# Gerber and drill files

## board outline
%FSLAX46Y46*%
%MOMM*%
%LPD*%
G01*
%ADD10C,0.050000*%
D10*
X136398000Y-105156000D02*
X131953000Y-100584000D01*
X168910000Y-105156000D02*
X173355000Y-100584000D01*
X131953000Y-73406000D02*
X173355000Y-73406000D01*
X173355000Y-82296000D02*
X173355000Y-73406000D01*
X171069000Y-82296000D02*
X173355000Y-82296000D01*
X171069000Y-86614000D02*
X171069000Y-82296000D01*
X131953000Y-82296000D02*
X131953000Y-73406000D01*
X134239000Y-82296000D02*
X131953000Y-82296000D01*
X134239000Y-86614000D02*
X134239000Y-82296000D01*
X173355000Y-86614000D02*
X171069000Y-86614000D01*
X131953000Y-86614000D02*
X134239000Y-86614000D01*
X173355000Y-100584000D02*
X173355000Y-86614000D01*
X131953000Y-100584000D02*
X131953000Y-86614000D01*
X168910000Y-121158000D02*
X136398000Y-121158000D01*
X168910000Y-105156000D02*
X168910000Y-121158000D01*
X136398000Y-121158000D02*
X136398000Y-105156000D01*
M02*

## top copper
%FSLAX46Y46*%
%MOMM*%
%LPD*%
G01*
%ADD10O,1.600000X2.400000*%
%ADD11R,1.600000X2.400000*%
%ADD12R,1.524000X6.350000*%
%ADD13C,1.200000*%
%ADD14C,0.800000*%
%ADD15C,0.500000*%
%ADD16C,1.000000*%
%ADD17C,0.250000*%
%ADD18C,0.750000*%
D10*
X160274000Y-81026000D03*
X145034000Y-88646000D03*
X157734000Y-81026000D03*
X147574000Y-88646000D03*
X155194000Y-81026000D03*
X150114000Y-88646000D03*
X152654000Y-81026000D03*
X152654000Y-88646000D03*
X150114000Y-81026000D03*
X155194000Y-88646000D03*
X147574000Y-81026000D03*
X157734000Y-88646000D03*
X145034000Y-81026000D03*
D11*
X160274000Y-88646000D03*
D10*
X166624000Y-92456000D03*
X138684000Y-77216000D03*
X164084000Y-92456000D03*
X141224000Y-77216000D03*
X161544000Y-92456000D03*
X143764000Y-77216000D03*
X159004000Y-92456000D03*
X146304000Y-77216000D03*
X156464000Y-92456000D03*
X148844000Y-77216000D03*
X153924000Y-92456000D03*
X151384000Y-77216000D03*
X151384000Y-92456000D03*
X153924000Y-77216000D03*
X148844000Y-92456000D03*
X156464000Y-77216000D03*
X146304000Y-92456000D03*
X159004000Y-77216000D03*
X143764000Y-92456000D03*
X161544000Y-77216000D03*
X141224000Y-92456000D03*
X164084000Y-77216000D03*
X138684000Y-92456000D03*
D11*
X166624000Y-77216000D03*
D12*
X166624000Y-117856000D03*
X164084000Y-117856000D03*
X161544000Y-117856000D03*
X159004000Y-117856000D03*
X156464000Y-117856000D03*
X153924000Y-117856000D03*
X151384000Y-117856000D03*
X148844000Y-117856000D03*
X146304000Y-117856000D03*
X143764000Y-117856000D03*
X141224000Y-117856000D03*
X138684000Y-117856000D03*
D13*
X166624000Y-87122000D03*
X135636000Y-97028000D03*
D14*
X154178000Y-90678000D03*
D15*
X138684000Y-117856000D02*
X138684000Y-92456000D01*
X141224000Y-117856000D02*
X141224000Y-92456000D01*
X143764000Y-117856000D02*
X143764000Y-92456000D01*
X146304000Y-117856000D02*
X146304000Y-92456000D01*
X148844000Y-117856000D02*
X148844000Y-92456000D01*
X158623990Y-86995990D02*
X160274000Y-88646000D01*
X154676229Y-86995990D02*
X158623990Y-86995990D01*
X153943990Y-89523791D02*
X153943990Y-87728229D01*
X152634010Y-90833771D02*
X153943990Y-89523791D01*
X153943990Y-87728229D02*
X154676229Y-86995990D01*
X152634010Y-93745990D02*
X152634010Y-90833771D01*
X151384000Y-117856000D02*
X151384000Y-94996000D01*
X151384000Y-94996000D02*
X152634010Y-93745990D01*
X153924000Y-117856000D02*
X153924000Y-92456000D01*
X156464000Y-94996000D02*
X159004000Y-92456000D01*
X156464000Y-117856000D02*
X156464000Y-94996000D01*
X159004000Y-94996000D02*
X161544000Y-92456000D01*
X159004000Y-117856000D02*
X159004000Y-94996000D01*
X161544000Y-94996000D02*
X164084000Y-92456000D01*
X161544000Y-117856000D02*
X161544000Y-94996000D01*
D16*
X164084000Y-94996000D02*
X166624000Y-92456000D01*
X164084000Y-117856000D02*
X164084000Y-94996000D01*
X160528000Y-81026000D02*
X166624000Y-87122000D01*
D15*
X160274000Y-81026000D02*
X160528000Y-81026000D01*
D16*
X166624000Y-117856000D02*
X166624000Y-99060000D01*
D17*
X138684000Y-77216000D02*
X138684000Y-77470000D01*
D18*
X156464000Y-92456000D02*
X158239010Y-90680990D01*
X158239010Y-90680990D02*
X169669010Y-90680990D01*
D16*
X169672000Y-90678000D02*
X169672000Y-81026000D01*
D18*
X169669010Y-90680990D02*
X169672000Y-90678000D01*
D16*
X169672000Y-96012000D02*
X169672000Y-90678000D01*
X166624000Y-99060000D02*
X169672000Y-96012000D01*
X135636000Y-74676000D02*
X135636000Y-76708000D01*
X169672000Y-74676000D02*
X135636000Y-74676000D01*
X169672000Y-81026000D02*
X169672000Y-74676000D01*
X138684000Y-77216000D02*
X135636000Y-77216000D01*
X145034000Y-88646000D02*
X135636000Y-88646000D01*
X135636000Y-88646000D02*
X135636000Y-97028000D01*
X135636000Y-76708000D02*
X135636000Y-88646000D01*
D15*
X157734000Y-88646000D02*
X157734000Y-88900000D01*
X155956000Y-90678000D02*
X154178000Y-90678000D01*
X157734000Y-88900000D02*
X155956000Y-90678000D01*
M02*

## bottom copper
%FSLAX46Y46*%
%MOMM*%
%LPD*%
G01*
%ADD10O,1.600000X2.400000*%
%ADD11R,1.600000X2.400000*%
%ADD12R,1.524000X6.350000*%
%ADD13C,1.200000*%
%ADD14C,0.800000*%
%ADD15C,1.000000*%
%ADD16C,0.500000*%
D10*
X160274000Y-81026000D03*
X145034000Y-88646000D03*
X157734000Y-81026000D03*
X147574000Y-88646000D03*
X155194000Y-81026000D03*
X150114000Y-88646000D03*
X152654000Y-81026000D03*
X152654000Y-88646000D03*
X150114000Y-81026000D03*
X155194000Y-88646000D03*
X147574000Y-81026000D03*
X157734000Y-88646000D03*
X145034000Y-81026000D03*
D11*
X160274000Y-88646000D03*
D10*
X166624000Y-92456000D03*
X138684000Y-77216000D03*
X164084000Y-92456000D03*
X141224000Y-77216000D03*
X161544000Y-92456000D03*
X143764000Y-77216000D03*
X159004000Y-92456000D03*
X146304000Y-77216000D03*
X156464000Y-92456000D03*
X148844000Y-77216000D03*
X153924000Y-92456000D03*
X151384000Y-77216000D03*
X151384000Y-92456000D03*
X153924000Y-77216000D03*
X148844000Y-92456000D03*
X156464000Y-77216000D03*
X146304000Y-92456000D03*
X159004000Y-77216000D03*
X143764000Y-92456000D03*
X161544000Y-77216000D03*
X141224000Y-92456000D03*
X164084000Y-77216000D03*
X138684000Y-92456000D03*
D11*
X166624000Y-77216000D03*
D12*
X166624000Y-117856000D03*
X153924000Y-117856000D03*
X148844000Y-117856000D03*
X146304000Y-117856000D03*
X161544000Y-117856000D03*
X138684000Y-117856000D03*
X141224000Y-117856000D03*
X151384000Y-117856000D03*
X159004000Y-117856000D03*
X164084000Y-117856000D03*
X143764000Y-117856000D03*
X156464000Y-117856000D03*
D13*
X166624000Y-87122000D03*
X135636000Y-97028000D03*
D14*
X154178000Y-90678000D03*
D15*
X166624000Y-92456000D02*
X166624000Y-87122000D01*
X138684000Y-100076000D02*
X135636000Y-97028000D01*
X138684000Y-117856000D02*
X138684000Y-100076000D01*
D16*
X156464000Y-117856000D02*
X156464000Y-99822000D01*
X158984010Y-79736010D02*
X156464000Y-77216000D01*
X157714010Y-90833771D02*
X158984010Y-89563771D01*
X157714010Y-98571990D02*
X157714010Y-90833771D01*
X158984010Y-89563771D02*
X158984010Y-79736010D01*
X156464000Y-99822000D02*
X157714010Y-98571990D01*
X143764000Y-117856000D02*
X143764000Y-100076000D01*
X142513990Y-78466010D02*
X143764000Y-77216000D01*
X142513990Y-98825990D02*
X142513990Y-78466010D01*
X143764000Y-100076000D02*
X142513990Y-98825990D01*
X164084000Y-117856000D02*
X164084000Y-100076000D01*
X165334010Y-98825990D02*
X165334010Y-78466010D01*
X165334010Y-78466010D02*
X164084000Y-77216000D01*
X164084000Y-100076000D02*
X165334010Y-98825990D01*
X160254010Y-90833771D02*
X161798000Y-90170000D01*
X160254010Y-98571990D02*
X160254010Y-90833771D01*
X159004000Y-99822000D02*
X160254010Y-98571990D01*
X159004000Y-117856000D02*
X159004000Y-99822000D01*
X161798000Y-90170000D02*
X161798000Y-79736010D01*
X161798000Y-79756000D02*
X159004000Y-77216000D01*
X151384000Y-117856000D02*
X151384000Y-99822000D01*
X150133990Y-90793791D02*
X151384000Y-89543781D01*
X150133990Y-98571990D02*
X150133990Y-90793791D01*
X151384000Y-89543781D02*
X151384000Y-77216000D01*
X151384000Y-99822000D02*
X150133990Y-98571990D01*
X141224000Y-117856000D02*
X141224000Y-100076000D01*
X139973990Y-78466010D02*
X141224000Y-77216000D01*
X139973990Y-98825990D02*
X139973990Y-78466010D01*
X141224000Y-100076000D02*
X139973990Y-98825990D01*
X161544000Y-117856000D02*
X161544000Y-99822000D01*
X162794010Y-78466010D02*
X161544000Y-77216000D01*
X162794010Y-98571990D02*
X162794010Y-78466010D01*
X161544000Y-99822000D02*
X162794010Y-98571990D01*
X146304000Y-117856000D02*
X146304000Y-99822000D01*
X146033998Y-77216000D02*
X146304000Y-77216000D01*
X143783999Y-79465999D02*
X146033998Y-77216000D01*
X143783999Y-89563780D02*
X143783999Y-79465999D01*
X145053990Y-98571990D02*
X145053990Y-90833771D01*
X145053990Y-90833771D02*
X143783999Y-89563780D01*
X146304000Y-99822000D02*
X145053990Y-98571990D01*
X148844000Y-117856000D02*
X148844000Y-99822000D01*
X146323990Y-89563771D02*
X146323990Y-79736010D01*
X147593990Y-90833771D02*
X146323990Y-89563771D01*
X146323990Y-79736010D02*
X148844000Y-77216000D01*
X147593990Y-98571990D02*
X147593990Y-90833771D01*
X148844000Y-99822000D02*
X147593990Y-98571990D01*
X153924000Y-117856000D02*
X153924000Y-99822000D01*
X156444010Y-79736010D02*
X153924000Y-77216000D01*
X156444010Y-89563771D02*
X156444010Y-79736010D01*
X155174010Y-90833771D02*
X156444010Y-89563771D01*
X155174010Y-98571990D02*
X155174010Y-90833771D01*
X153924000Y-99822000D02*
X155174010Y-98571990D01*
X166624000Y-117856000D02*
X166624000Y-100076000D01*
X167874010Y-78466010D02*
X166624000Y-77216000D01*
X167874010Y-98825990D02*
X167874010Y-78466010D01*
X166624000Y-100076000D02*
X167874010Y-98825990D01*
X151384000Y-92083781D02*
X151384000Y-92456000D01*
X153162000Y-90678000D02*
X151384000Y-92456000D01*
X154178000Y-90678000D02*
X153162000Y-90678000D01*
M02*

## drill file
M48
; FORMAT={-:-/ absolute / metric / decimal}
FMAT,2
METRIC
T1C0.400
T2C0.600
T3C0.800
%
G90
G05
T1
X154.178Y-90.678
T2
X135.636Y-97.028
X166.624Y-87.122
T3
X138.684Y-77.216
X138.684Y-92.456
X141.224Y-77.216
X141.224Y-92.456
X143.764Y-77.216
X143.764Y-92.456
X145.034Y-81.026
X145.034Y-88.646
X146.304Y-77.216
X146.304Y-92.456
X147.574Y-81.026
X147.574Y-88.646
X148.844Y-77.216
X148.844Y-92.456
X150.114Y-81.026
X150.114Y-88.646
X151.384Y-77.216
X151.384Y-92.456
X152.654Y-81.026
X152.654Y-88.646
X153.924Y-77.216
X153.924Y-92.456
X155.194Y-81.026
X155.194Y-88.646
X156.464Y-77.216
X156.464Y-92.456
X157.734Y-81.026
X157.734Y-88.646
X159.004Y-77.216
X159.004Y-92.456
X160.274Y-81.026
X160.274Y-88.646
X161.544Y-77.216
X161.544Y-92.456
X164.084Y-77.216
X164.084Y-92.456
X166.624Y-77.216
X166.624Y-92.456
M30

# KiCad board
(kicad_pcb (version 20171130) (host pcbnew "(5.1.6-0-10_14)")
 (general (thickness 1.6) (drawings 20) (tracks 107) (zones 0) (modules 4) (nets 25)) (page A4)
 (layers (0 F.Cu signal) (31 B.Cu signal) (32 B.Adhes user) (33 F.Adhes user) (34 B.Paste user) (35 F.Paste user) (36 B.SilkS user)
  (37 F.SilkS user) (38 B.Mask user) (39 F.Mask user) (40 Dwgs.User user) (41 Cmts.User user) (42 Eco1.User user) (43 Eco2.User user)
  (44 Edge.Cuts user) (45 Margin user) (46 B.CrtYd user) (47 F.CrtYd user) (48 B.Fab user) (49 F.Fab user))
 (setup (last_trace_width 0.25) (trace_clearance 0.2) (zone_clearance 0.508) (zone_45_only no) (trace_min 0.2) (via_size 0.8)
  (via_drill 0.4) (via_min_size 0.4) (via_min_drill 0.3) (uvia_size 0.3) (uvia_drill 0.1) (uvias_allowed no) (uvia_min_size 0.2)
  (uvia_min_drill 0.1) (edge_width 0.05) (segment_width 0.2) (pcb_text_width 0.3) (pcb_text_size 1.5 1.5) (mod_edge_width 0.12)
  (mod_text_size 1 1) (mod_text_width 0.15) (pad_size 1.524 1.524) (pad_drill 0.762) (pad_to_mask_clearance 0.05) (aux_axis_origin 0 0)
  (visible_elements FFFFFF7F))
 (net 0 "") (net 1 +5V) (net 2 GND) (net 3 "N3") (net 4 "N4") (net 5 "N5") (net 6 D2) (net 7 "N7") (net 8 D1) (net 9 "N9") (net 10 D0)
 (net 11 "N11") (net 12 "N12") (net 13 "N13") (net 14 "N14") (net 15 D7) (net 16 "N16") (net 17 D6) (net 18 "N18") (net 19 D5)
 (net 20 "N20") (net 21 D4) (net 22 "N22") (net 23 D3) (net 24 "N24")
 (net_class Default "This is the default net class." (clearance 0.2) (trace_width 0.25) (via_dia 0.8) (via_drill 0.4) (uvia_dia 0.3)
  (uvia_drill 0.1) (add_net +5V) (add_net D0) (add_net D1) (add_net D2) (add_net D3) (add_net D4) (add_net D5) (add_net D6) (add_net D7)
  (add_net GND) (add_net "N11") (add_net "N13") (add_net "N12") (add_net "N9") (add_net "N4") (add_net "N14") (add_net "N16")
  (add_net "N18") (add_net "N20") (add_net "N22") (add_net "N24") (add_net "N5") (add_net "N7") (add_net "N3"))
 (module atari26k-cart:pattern (layer F.Cu) (at 152.654 105.41)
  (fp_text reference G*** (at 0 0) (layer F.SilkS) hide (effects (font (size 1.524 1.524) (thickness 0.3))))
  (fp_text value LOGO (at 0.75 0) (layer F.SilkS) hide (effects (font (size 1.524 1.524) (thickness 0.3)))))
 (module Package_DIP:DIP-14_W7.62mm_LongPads (layer B.Cu) (at 160.274 88.646 90)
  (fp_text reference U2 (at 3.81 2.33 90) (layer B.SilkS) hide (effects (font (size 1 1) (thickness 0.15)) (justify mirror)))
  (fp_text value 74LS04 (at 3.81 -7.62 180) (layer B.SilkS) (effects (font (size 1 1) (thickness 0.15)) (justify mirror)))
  (pad 14 thru_hole oval (at 7.62 0 90) (size 2.4 1.6) (drill 0.8) (layers *.Cu *.Mask) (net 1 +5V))
  (pad 7 thru_hole oval (at 0 -15.24 90) (size 2.4 1.6) (drill 0.8) (layers *.Cu *.Mask) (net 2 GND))
  (pad 13 thru_hole oval (at 7.62 -2.54 90) (size 2.4 1.6) (drill 0.8) (layers *.Cu *.Mask))
  (pad 6 thru_hole oval (at 0 -12.7 90) (size 2.4 1.6) (drill 0.8) (layers *.Cu *.Mask))
  (pad 12 thru_hole oval (at 7.62 -5.08 90) (size 2.4 1.6) (drill 0.8) (layers *.Cu *.Mask))
  (pad 5 thru_hole oval (at 0 -10.16 90) (size 2.4 1.6) (drill 0.8) (layers *.Cu *.Mask))
  (pad 11 thru_hole oval (at 7.62 -7.62 90) (size 2.4 1.6) (drill 0.8) (layers *.Cu *.Mask))
  (pad 4 thru_hole oval (at 0 -7.62 90) (size 2.4 1.6) (drill 0.8) (layers *.Cu *.Mask))
  (pad 10 thru_hole oval (at 7.62 -10.16 90) (size 2.4 1.6) (drill 0.8) (layers *.Cu *.Mask))
  (pad 3 thru_hole oval (at 0 -5.08 90) (size 2.4 1.6) (drill 0.8) (layers *.Cu *.Mask))
  (pad 9 thru_hole oval (at 7.62 -12.7 90) (size 2.4 1.6) (drill 0.8) (layers *.Cu *.Mask))
  (pad 2 thru_hole oval (at 0 -2.54 90) (size 2.4 1.6) (drill 0.8) (layers *.Cu *.Mask) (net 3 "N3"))
  (pad 8 thru_hole oval (at 7.62 -15.24 90) (size 2.4 1.6) (drill 0.8) (layers *.Cu *.Mask))
  (pad 1 thru_hole rect (at 0 0 90) (size 2.4 1.6) (drill 0.8) (layers *.Cu *.Mask) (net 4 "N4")))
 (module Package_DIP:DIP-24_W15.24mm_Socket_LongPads (layer F.Cu) (at 166.624 77.216 270)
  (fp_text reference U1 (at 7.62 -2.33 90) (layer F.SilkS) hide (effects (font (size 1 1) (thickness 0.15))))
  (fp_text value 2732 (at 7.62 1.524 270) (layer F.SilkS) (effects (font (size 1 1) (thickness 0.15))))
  (pad 24 thru_hole oval (at 15.24 0 270) (size 2.4 1.6) (drill 0.8) (layers *.Cu *.Mask) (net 1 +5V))
  (pad 12 thru_hole oval (at 0 27.94 270) (size 2.4 1.6) (drill 0.8) (layers *.Cu *.Mask) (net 2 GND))
  (pad 23 thru_hole oval (at 15.24 2.54 270) (size 2.4 1.6) (drill 0.8) (layers *.Cu *.Mask) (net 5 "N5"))
  (pad 11 thru_hole oval (at 0 25.4 270) (size 2.4 1.6) (drill 0.8) (layers *.Cu *.Mask) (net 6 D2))
  (pad 22 thru_hole oval (at 15.24 5.08 270) (size 2.4 1.6) (drill 0.8) (layers *.Cu *.Mask) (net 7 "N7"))
  (pad 10 thru_hole oval (at 0 22.86 270) (size 2.4 1.6) (drill 0.8) (layers *.Cu *.Mask) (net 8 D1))
  (pad 21 thru_hole oval (at 15.24 7.62 270) (size 2.4 1.6) (drill 0.8) (layers *.Cu *.Mask) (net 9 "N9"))
  (pad 9 thru_hole oval (at 0 20.32 270) (size 2.4 1.6) (drill 0.8) (layers *.Cu *.Mask) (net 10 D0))
  (pad 20 thru_hole oval (at 15.24 10.16 270) (size 2.4 1.6) (drill 0.8) (layers *.Cu *.Mask) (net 2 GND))
  (pad 8 thru_hole oval (at 0 17.78 270) (size 2.4 1.6) (drill 0.8) (layers *.Cu *.Mask) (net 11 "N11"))
  (pad 19 thru_hole oval (at 15.24 12.7 270) (size 2.4 1.6) (drill 0.8) (layers *.Cu *.Mask) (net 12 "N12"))
  (pad 7 thru_hole oval (at 0 15.24 270) (size 2.4 1.6) (drill 0.8) (layers *.Cu *.Mask) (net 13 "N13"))
  (pad 18 thru_hole oval (at 15.24 15.24 270) (size 2.4 1.6) (drill 0.8) (layers *.Cu *.Mask) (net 3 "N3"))
  (pad 6 thru_hole oval (at 0 12.7 270) (size 2.4 1.6) (drill 0.8) (layers *.Cu *.Mask) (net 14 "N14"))
  (pad 17 thru_hole oval (at 15.24 17.78 270) (size 2.4 1.6) (drill 0.8) (layers *.Cu *.Mask) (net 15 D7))
  (pad 5 thru_hole oval (at 0 10.16 270) (size 2.4 1.6) (drill 0.8) (layers *.Cu *.Mask) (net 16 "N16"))
  (pad 16 thru_hole oval (at 15.24 20.32 270) (size 2.4 1.6) (drill 0.8) (layers *.Cu *.Mask) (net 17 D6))
  (pad 4 thru_hole oval (at 0 7.62 270) (size 2.4 1.6) (drill 0.8) (layers *.Cu *.Mask) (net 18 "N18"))
  (pad 15 thru_hole oval (at 15.24 22.86 270) (size 2.4 1.6) (drill 0.8) (layers *.Cu *.Mask) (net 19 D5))
  (pad 3 thru_hole oval (at 0 5.08 270) (size 2.4 1.6) (drill 0.8) (layers *.Cu *.Mask) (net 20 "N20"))
  (pad 14 thru_hole oval (at 15.24 25.4 270) (size 2.4 1.6) (drill 0.8) (layers *.Cu *.Mask) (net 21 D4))
  (pad 2 thru_hole oval (at 0 2.54 270) (size 2.4 1.6) (drill 0.8) (layers *.Cu *.Mask) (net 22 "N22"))
  (pad 13 thru_hole oval (at 15.24 27.94 270) (size 2.4 1.6) (drill 0.8) (layers *.Cu *.Mask) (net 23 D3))
  (pad 1 thru_hole rect (at 0 0 270) (size 2.4 1.6) (drill 0.8) (layers *.Cu *.Mask) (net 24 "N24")))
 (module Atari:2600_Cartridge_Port (layer F.Cu) (at 138.176 114.808)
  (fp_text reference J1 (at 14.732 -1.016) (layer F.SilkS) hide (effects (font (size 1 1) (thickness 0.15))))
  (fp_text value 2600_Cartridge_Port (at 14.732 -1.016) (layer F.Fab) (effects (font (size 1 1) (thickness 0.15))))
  (pad A7 connect rect (at 28.448 3.048) (size 1.524 6.35) (layers B.Cu B.Mask) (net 24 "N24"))
  (pad A2 connect rect (at 15.748 3.048) (size 1.524 6.35) (layers B.Cu B.Mask) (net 14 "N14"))
  (pad A0 connect rect (at 10.668 3.048) (size 1.524 6.35) (layers B.Cu B.Mask) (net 11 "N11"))
  (pad D0 connect rect (at 8.128 3.048) (size 1.524 6.35) (layers B.Cu B.Mask) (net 10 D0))
  (pad A5 connect rect (at 23.368 3.048) (size 1.524 6.35) (layers B.Cu B.Mask) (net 20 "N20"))
  (pad GND connect rect (at 0.508 3.048) (size 1.524 6.35) (layers B.Cu B.Mask) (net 2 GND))
  (pad D2 connect rect (at 3.048 3.048) (size 1.524 6.35) (layers B.Cu B.Mask) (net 6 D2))
  (pad A1 connect rect (at 13.208 3.048) (size 1.524 6.35) (layers B.Cu B.Mask) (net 13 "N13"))
  (pad A4 connect rect (at 20.828 3.048) (size 1.524 6.35) (layers B.Cu B.Mask) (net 18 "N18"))
  (pad A6 connect rect (at 25.908 3.048) (size 1.524 6.35) (layers B.Cu B.Mask) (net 22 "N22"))
  (pad D1 connect rect (at 5.588 3.048) (size 1.524 6.35) (layers B.Cu B.Mask) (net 8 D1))
  (pad A3 connect rect (at 18.288 3.048) (size 1.524 6.35) (layers B.Cu B.Mask) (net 16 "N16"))
  (pad SGND connect rect (at 28.448 3.048) (size 1.524 6.35) (layers F.Cu F.Mask) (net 2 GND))
  (pad +5V connect rect (at 25.908 3.048) (size 1.524 6.35) (layers F.Cu F.Mask) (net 1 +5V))
  (pad A8 connect rect (at 23.368 3.048) (size 1.524 6.35) (layers F.Cu F.Mask) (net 5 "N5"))
  (pad A9 connect rect (at 20.828 3.048) (size 1.524 6.35) (layers F.Cu F.Mask) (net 7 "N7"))
  (pad A11 connect rect (at 18.288 3.048) (size 1.524 6.35) (layers F.Cu F.Mask) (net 9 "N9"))
  (pad A10 connect rect (at 15.748 3.048) (size 1.524 6.35) (layers F.Cu F.Mask) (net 12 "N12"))
  (pad A12 connect rect (at 13.208 3.048) (size 1.524 6.35) (layers F.Cu F.Mask) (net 4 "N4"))
  (pad D7 connect rect (at 10.668 3.048) (size 1.524 6.35) (layers F.Cu F.Mask) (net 15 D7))
  (pad D6 connect rect (at 8.128 3.048) (size 1.524 6.35) (layers F.Cu F.Mask) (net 17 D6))
  (pad D5 connect rect (at 5.588 3.048) (size 1.524 6.35) (layers F.Cu F.Mask) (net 19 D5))
  (pad D4 connect rect (at 3.048 3.048) (size 1.524 6.35) (layers F.Cu F.Mask) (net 21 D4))
  (pad D3 connect rect (at 0.508 3.048) (size 1.524 6.35) (layers F.Cu F.Mask) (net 23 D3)))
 (gr_line (start 136.398 105.156) (end 131.953 100.584) (layer Edge.Cuts) (width 0.05))
 (gr_line (start 168.91 105.156) (end 173.355 100.584) (layer Edge.Cuts) (width 0.05))
 (gr_line (start 131.953 73.406) (end 173.355 73.406) (layer Edge.Cuts) (width 0.05))
 (gr_line (start 173.355 82.296) (end 173.355 73.406) (layer Edge.Cuts) (width 0.05))
 (gr_line (start 171.069 82.296) (end 173.355 82.296) (layer Edge.Cuts) (width 0.05))
 (gr_line (start 171.069 86.614) (end 171.069 82.296) (layer Edge.Cuts) (width 0.05))
 (gr_line (start 131.953 82.296) (end 131.953 73.406) (layer Edge.Cuts) (width 0.05))
 (gr_line (start 134.239 82.296) (end 131.953 82.296) (layer Edge.Cuts) (width 0.05))
 (gr_line (start 134.239 86.614) (end 134.239 82.296) (layer Edge.Cuts) (width 0.05))
 (gr_line (start 173.355 86.614) (end 171.069 86.614) (layer Edge.Cuts) (width 0.05))
 (gr_line (start 131.953 86.614) (end 134.239 86.614) (layer Edge.Cuts) (width 0.05))
 (gr_line (start 173.355 100.584) (end 173.355 86.614) (layer Edge.Cuts) (width 0.05))
 (gr_line (start 131.953 100.584) (end 131.953 86.614) (layer Edge.Cuts) (width 0.05))
 (gr_line (start 168.91 121.158) (end 136.398 121.158) (layer Edge.Cuts) (width 0.05))
 (gr_line (start 168.91 105.156) (end 168.91 121.158) (layer Edge.Cuts) (width 0.05))
 (gr_line (start 136.398 121.158) (end 136.398 105.156) (layer Edge.Cuts) (width 0.05))
 (segment (start 138.684 117.856) (end 138.684 92.456) (width 0.5) (layer F.Cu) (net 23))
 (segment (start 141.224 117.856) (end 141.224 92.456) (width 0.5) (layer F.Cu) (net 21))
 (segment (start 143.764 117.856) (end 143.764 92.456) (width 0.5) (layer F.Cu) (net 19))
 (segment (start 146.304 117.856) (end 146.304 92.456) (width 0.5) (layer F.Cu) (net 17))
 (segment (start 148.844 117.856) (end 148.844 92.456) (width 0.5) (layer F.Cu) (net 15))
 (segment (start 158.62399 86.99599) (end 160.274 88.646) (width 0.5) (layer F.Cu) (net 4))
 (segment (start 154.676229 86.99599) (end 158.62399 86.99599) (width 0.5) (layer F.Cu) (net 4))
 (segment (start 153.94399 89.523791) (end 153.94399 87.728229) (width 0.5) (layer F.Cu) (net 4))
 (segment (start 152.63401 90.833771) (end 153.94399 89.523791) (width 0.5) (layer F.Cu) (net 4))
 (segment (start 153.94399 87.728229) (end 154.676229 86.99599) (width 0.5) (layer F.Cu) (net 4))
 (segment (start 152.63401 93.74599) (end 152.63401 90.833771) (width 0.5) (layer F.Cu) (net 4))
 (segment (start 151.384 117.856) (end 151.384 94.996) (width 0.5) (layer F.Cu) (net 4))
 (segment (start 151.384 94.996) (end 152.63401 93.74599) (width 0.5) (layer F.Cu) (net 4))
 (segment (start 153.924 117.856) (end 153.924 92.456) (width 0.5) (layer F.Cu) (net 12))
 (segment (start 156.464 94.996) (end 159.004 92.456) (width 0.5) (layer F.Cu) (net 9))
 (segment (start 156.464 117.856) (end 156.464 94.996) (width 0.5) (layer F.Cu) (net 9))
 (segment (start 159.004 94.996) (end 161.544 92.456) (width 0.5) (layer F.Cu) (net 7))
 (segment (start 159.004 117.856) (end 159.004 94.996) (width 0.5) (layer F.Cu) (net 7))
 (segment (start 161.544 94.996) (end 164.084 92.456) (width 0.5) (layer F.Cu) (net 5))
 (segment (start 161.544 117.856) (end 161.544 94.996) (width 0.5) (layer F.Cu) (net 5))
 (segment (start 164.084 94.996) (end 166.624 92.456) (width 1) (layer F.Cu) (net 1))
 (segment (start 164.084 117.856) (end 164.084 94.996) (width 1) (layer F.Cu) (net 1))
 (via (at 166.624 87.122) (size 1.2) (drill 0.6) (layers F.Cu B.Cu) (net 1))
 (segment (start 166.624 92.456) (end 166.624 87.122) (width 1) (layer B.Cu) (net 1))
 (segment (start 160.528 81.026) (end 166.624 87.122) (width 1) (layer F.Cu) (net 1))
 (segment (start 160.274 81.026) (end 160.528 81.026) (width 0.5) (layer F.Cu) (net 1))
 (segment (start 166.624 117.856) (end 166.624 99.06) (width 1) (layer F.Cu) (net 2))
 (segment (start 138.684 77.216) (end 138.684 77.47) (width 0.25) (layer F.Cu) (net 2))
 (segment (start 156.464 92.456) (end 158.23901 90.68099) (width 0.75) (layer F.Cu) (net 2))
 (segment (start 158.23901 90.68099) (end 169.66901 90.68099) (width 0.75) (layer F.Cu) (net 2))
 (segment (start 169.672 90.678) (end 169.672 81.026) (width 1) (layer F.Cu) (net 2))
 (segment (start 169.66901 90.68099) (end 169.672 90.678) (width 0.75) (layer F.Cu) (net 2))
 (via (at 135.636 97.028) (size 1.2) (drill 0.6) (layers F.Cu B.Cu) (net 2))
 (segment (start 169.672 96.012) (end 169.672 90.678) (width 1) (layer F.Cu) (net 2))
 (segment (start 166.624 99.06) (end 169.672 96.012) (width 1) (layer F.Cu) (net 2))
 (segment (start 135.636 74.676) (end 135.636 76.708) (width 1) (layer F.Cu) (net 2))
 (segment (start 138.684 100.076) (end 135.636 97.028) (width 1) (layer B.Cu) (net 2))
 (segment (start 138.684 117.856) (end 138.684 100.076) (width 1) (layer B.Cu) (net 2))
 (segment (start 169.672 74.676) (end 135.636 74.676) (width 1) (layer F.Cu) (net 2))
 (segment (start 169.672 81.026) (end 169.672 74.676) (width 1) (layer F.Cu) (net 2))
 (segment (start 138.684 77.216) (end 135.636 77.216) (width 1) (layer F.Cu) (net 2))
 (segment (start 145.034 88.646) (end 135.636 88.646) (width 1) (layer F.Cu) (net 2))
 (segment (start 135.636 88.646) (end 135.636 97.028) (width 1) (layer F.Cu) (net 2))
 (segment (start 135.636 76.708) (end 135.636 88.646) (width 1) (layer F.Cu) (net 2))
 (segment (start 156.464 117.856) (end 156.464 99.822) (width 0.5) (layer B.Cu) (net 16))
 (segment (start 158.98401 79.73601) (end 156.464 77.216) (width 0.5) (layer B.Cu) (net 16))
 (segment (start 157.71401 90.833771) (end 158.98401 89.563771) (width 0.5) (layer B.Cu) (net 16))
 (segment (start 157.71401 98.57199) (end 157.71401 90.833771) (width 0.5) (layer B.Cu) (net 16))
 (segment (start 158.98401 89.563771) (end 158.98401 79.73601) (width 0.5) (layer B.Cu) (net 16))
 (segment (start 156.464 99.822) (end 157.71401 98.57199) (width 0.5) (layer B.Cu) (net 16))
 (segment (start 143.764 117.856) (end 143.764 100.076) (width 0.5) (layer B.Cu) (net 8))
 (segment (start 142.51399 78.46601) (end 143.764 77.216) (width 0.5) (layer B.Cu) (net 8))
 (segment (start 142.51399 98.82599) (end 142.51399 78.46601) (width 0.5) (layer B.Cu) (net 8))
 (segment (start 143.764 100.076) (end 142.51399 98.82599) (width 0.5) (layer B.Cu) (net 8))
 (segment (start 164.084 117.856) (end 164.084 100.076) (width 0.5) (layer B.Cu) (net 22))
 (segment (start 165.33401 98.82599) (end 165.33401 78.46601) (width 0.5) (layer B.Cu) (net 22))
 (segment (start 165.33401 78.46601) (end 164.084 77.216) (width 0.5) (layer B.Cu) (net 22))
 (segment (start 164.084 100.076) (end 165.33401 98.82599) (width 0.5) (layer B.Cu) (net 22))
 (segment (start 160.25401 90.833771) (end 161.798 90.17) (width 0.5) (layer B.Cu) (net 18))
 (segment (start 160.25401 98.57199) (end 160.25401 90.833771) (width 0.5) (layer B.Cu) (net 18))
 (segment (start 159.004 99.822) (end 160.25401 98.57199) (width 0.5) (layer B.Cu) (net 18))
 (segment (start 159.004 117.856) (end 159.004 99.822) (width 0.5) (layer B.Cu) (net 18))
 (segment (start 161.798 90.17) (end 161.798 79.73601) (width 0.5) (layer B.Cu) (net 18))
 (segment (start 161.798 79.756) (end 159.004 77.216) (width 0.5) (layer B.Cu) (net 18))
 (segment (start 151.384 117.856) (end 151.384 99.822) (width 0.5) (layer B.Cu) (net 13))
 (segment (start 150.13399 90.793791) (end 151.384 89.543781) (width 0.5) (layer B.Cu) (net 13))
 (segment (start 150.13399 98.57199) (end 150.13399 90.793791) (width 0.5) (layer B.Cu) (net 13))
 (segment (start 151.384 89.543781) (end 151.384 77.216) (width 0.5) (layer B.Cu) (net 13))
 (segment (start 151.384 99.822) (end 150.13399 98.57199) (width 0.5) (layer B.Cu) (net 13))
 (segment (start 141.224 117.856) (end 141.224 100.076) (width 0.5) (layer B.Cu) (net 6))
 (segment (start 139.97399 78.46601) (end 141.224 77.216) (width 0.5) (layer B.Cu) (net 6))
 (segment (start 139.97399 98.82599) (end 139.97399 78.46601) (width 0.5) (layer B.Cu) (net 6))
 (segment (start 141.224 100.076) (end 139.97399 98.82599) (width 0.5) (layer B.Cu) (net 6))
 (segment (start 161.544 117.856) (end 161.544 99.822) (width 0.5) (layer B.Cu) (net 20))
 (segment (start 162.79401 78.46601) (end 161.544 77.216) (width 0.5) (layer B.Cu) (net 20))
 (segment (start 162.79401 98.57199) (end 162.79401 78.46601) (width 0.5) (layer B.Cu) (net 20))
 (segment (start 161.544 99.822) (end 162.79401 98.57199) (width 0.5) (layer B.Cu) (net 20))
 (segment (start 146.304 117.856) (end 146.304 99.822) (width 0.5) (layer B.Cu) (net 10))
 (segment (start 146.033998 77.216) (end 146.304 77.216) (width 0.5) (layer B.Cu) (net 10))
 (segment (start 143.783999 79.465999) (end 146.033998 77.216) (width 0.5) (layer B.Cu) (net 10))
 (segment (start 143.783999 89.56378) (end 143.783999 79.465999) (width 0.5) (layer B.Cu) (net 10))
 (segment (start 145.05399 98.57199) (end 145.05399 90.833771) (width 0.5) (layer B.Cu) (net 10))
 (segment (start 145.05399 90.833771) (end 143.783999 89.56378) (width 0.5) (layer B.Cu) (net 10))
 (segment (start 146.304 99.822) (end 145.05399 98.57199) (width 0.5) (layer B.Cu) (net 10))
 (segment (start 148.844 117.856) (end 148.844 99.822) (width 0.5) (layer B.Cu) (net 11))
 (segment (start 146.32399 89.563771) (end 146.32399 79.73601) (width 0.5) (layer B.Cu) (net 11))
 (segment (start 147.59399 90.833771) (end 146.32399 89.563771) (width 0.5) (layer B.Cu) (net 11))
 (segment (start 146.32399 79.73601) (end 148.844 77.216) (width 0.5) (layer B.Cu) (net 11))
 (segment (start 147.59399 98.57199) (end 147.59399 90.833771) (width 0.5) (layer B.Cu) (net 11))
 (segment (start 148.844 99.822) (end 147.59399 98.57199) (width 0.5) (layer B.Cu) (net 11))
 (segment (start 153.924 117.856) (end 153.924 99.822) (width 0.5) (layer B.Cu) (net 14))
 (segment (start 156.44401 79.73601) (end 153.924 77.216) (width 0.5) (layer B.Cu) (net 14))
 (segment (start 156.44401 89.563771) (end 156.44401 79.73601) (width 0.5) (layer B.Cu) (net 14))
 (segment (start 155.17401 90.833771) (end 156.44401 89.563771) (width 0.5) (layer B.Cu) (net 14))
 (segment (start 155.17401 98.57199) (end 155.17401 90.833771) (width 0.5) (layer B.Cu) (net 14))
 (segment (start 153.924 99.822) (end 155.17401 98.57199) (width 0.5) (layer B.Cu) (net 14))
 (segment (start 166.624 117.856) (end 166.624 100.076) (width 0.5) (layer B.Cu) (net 24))
 (segment (start 167.87401 78.46601) (end 166.624 77.216) (width 0.5) (layer B.Cu) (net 24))
 (segment (start 167.87401 98.82599) (end 167.87401 78.46601) (width 0.5) (layer B.Cu) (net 24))
 (segment (start 166.624 100.076) (end 167.87401 98.82599) (width 0.5) (layer B.Cu) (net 24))
 (segment (start 151.384 92.083781) (end 151.384 92.456) (width 0.5) (layer B.Cu) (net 3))
 (segment (start 157.734 88.646) (end 157.734 88.9) (width 0.5) (layer F.Cu) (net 3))
 (via (at 154.178 90.678) (size 0.8) (drill 0.4) (layers F.Cu B.Cu) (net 3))
 (segment (start 155.956 90.678) (end 154.178 90.678) (width 0.5) (layer F.Cu) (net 3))
 (segment (start 157.734 88.9) (end 155.956 90.678) (width 0.5) (layer F.Cu) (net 3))
 (segment (start 153.162 90.678) (end 151.384 92.456) (width 0.5) (layer B.Cu) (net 3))
 (segment (start 154.178 90.678) (end 153.162 90.678) (width 0.5) (layer B.Cu) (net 3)))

